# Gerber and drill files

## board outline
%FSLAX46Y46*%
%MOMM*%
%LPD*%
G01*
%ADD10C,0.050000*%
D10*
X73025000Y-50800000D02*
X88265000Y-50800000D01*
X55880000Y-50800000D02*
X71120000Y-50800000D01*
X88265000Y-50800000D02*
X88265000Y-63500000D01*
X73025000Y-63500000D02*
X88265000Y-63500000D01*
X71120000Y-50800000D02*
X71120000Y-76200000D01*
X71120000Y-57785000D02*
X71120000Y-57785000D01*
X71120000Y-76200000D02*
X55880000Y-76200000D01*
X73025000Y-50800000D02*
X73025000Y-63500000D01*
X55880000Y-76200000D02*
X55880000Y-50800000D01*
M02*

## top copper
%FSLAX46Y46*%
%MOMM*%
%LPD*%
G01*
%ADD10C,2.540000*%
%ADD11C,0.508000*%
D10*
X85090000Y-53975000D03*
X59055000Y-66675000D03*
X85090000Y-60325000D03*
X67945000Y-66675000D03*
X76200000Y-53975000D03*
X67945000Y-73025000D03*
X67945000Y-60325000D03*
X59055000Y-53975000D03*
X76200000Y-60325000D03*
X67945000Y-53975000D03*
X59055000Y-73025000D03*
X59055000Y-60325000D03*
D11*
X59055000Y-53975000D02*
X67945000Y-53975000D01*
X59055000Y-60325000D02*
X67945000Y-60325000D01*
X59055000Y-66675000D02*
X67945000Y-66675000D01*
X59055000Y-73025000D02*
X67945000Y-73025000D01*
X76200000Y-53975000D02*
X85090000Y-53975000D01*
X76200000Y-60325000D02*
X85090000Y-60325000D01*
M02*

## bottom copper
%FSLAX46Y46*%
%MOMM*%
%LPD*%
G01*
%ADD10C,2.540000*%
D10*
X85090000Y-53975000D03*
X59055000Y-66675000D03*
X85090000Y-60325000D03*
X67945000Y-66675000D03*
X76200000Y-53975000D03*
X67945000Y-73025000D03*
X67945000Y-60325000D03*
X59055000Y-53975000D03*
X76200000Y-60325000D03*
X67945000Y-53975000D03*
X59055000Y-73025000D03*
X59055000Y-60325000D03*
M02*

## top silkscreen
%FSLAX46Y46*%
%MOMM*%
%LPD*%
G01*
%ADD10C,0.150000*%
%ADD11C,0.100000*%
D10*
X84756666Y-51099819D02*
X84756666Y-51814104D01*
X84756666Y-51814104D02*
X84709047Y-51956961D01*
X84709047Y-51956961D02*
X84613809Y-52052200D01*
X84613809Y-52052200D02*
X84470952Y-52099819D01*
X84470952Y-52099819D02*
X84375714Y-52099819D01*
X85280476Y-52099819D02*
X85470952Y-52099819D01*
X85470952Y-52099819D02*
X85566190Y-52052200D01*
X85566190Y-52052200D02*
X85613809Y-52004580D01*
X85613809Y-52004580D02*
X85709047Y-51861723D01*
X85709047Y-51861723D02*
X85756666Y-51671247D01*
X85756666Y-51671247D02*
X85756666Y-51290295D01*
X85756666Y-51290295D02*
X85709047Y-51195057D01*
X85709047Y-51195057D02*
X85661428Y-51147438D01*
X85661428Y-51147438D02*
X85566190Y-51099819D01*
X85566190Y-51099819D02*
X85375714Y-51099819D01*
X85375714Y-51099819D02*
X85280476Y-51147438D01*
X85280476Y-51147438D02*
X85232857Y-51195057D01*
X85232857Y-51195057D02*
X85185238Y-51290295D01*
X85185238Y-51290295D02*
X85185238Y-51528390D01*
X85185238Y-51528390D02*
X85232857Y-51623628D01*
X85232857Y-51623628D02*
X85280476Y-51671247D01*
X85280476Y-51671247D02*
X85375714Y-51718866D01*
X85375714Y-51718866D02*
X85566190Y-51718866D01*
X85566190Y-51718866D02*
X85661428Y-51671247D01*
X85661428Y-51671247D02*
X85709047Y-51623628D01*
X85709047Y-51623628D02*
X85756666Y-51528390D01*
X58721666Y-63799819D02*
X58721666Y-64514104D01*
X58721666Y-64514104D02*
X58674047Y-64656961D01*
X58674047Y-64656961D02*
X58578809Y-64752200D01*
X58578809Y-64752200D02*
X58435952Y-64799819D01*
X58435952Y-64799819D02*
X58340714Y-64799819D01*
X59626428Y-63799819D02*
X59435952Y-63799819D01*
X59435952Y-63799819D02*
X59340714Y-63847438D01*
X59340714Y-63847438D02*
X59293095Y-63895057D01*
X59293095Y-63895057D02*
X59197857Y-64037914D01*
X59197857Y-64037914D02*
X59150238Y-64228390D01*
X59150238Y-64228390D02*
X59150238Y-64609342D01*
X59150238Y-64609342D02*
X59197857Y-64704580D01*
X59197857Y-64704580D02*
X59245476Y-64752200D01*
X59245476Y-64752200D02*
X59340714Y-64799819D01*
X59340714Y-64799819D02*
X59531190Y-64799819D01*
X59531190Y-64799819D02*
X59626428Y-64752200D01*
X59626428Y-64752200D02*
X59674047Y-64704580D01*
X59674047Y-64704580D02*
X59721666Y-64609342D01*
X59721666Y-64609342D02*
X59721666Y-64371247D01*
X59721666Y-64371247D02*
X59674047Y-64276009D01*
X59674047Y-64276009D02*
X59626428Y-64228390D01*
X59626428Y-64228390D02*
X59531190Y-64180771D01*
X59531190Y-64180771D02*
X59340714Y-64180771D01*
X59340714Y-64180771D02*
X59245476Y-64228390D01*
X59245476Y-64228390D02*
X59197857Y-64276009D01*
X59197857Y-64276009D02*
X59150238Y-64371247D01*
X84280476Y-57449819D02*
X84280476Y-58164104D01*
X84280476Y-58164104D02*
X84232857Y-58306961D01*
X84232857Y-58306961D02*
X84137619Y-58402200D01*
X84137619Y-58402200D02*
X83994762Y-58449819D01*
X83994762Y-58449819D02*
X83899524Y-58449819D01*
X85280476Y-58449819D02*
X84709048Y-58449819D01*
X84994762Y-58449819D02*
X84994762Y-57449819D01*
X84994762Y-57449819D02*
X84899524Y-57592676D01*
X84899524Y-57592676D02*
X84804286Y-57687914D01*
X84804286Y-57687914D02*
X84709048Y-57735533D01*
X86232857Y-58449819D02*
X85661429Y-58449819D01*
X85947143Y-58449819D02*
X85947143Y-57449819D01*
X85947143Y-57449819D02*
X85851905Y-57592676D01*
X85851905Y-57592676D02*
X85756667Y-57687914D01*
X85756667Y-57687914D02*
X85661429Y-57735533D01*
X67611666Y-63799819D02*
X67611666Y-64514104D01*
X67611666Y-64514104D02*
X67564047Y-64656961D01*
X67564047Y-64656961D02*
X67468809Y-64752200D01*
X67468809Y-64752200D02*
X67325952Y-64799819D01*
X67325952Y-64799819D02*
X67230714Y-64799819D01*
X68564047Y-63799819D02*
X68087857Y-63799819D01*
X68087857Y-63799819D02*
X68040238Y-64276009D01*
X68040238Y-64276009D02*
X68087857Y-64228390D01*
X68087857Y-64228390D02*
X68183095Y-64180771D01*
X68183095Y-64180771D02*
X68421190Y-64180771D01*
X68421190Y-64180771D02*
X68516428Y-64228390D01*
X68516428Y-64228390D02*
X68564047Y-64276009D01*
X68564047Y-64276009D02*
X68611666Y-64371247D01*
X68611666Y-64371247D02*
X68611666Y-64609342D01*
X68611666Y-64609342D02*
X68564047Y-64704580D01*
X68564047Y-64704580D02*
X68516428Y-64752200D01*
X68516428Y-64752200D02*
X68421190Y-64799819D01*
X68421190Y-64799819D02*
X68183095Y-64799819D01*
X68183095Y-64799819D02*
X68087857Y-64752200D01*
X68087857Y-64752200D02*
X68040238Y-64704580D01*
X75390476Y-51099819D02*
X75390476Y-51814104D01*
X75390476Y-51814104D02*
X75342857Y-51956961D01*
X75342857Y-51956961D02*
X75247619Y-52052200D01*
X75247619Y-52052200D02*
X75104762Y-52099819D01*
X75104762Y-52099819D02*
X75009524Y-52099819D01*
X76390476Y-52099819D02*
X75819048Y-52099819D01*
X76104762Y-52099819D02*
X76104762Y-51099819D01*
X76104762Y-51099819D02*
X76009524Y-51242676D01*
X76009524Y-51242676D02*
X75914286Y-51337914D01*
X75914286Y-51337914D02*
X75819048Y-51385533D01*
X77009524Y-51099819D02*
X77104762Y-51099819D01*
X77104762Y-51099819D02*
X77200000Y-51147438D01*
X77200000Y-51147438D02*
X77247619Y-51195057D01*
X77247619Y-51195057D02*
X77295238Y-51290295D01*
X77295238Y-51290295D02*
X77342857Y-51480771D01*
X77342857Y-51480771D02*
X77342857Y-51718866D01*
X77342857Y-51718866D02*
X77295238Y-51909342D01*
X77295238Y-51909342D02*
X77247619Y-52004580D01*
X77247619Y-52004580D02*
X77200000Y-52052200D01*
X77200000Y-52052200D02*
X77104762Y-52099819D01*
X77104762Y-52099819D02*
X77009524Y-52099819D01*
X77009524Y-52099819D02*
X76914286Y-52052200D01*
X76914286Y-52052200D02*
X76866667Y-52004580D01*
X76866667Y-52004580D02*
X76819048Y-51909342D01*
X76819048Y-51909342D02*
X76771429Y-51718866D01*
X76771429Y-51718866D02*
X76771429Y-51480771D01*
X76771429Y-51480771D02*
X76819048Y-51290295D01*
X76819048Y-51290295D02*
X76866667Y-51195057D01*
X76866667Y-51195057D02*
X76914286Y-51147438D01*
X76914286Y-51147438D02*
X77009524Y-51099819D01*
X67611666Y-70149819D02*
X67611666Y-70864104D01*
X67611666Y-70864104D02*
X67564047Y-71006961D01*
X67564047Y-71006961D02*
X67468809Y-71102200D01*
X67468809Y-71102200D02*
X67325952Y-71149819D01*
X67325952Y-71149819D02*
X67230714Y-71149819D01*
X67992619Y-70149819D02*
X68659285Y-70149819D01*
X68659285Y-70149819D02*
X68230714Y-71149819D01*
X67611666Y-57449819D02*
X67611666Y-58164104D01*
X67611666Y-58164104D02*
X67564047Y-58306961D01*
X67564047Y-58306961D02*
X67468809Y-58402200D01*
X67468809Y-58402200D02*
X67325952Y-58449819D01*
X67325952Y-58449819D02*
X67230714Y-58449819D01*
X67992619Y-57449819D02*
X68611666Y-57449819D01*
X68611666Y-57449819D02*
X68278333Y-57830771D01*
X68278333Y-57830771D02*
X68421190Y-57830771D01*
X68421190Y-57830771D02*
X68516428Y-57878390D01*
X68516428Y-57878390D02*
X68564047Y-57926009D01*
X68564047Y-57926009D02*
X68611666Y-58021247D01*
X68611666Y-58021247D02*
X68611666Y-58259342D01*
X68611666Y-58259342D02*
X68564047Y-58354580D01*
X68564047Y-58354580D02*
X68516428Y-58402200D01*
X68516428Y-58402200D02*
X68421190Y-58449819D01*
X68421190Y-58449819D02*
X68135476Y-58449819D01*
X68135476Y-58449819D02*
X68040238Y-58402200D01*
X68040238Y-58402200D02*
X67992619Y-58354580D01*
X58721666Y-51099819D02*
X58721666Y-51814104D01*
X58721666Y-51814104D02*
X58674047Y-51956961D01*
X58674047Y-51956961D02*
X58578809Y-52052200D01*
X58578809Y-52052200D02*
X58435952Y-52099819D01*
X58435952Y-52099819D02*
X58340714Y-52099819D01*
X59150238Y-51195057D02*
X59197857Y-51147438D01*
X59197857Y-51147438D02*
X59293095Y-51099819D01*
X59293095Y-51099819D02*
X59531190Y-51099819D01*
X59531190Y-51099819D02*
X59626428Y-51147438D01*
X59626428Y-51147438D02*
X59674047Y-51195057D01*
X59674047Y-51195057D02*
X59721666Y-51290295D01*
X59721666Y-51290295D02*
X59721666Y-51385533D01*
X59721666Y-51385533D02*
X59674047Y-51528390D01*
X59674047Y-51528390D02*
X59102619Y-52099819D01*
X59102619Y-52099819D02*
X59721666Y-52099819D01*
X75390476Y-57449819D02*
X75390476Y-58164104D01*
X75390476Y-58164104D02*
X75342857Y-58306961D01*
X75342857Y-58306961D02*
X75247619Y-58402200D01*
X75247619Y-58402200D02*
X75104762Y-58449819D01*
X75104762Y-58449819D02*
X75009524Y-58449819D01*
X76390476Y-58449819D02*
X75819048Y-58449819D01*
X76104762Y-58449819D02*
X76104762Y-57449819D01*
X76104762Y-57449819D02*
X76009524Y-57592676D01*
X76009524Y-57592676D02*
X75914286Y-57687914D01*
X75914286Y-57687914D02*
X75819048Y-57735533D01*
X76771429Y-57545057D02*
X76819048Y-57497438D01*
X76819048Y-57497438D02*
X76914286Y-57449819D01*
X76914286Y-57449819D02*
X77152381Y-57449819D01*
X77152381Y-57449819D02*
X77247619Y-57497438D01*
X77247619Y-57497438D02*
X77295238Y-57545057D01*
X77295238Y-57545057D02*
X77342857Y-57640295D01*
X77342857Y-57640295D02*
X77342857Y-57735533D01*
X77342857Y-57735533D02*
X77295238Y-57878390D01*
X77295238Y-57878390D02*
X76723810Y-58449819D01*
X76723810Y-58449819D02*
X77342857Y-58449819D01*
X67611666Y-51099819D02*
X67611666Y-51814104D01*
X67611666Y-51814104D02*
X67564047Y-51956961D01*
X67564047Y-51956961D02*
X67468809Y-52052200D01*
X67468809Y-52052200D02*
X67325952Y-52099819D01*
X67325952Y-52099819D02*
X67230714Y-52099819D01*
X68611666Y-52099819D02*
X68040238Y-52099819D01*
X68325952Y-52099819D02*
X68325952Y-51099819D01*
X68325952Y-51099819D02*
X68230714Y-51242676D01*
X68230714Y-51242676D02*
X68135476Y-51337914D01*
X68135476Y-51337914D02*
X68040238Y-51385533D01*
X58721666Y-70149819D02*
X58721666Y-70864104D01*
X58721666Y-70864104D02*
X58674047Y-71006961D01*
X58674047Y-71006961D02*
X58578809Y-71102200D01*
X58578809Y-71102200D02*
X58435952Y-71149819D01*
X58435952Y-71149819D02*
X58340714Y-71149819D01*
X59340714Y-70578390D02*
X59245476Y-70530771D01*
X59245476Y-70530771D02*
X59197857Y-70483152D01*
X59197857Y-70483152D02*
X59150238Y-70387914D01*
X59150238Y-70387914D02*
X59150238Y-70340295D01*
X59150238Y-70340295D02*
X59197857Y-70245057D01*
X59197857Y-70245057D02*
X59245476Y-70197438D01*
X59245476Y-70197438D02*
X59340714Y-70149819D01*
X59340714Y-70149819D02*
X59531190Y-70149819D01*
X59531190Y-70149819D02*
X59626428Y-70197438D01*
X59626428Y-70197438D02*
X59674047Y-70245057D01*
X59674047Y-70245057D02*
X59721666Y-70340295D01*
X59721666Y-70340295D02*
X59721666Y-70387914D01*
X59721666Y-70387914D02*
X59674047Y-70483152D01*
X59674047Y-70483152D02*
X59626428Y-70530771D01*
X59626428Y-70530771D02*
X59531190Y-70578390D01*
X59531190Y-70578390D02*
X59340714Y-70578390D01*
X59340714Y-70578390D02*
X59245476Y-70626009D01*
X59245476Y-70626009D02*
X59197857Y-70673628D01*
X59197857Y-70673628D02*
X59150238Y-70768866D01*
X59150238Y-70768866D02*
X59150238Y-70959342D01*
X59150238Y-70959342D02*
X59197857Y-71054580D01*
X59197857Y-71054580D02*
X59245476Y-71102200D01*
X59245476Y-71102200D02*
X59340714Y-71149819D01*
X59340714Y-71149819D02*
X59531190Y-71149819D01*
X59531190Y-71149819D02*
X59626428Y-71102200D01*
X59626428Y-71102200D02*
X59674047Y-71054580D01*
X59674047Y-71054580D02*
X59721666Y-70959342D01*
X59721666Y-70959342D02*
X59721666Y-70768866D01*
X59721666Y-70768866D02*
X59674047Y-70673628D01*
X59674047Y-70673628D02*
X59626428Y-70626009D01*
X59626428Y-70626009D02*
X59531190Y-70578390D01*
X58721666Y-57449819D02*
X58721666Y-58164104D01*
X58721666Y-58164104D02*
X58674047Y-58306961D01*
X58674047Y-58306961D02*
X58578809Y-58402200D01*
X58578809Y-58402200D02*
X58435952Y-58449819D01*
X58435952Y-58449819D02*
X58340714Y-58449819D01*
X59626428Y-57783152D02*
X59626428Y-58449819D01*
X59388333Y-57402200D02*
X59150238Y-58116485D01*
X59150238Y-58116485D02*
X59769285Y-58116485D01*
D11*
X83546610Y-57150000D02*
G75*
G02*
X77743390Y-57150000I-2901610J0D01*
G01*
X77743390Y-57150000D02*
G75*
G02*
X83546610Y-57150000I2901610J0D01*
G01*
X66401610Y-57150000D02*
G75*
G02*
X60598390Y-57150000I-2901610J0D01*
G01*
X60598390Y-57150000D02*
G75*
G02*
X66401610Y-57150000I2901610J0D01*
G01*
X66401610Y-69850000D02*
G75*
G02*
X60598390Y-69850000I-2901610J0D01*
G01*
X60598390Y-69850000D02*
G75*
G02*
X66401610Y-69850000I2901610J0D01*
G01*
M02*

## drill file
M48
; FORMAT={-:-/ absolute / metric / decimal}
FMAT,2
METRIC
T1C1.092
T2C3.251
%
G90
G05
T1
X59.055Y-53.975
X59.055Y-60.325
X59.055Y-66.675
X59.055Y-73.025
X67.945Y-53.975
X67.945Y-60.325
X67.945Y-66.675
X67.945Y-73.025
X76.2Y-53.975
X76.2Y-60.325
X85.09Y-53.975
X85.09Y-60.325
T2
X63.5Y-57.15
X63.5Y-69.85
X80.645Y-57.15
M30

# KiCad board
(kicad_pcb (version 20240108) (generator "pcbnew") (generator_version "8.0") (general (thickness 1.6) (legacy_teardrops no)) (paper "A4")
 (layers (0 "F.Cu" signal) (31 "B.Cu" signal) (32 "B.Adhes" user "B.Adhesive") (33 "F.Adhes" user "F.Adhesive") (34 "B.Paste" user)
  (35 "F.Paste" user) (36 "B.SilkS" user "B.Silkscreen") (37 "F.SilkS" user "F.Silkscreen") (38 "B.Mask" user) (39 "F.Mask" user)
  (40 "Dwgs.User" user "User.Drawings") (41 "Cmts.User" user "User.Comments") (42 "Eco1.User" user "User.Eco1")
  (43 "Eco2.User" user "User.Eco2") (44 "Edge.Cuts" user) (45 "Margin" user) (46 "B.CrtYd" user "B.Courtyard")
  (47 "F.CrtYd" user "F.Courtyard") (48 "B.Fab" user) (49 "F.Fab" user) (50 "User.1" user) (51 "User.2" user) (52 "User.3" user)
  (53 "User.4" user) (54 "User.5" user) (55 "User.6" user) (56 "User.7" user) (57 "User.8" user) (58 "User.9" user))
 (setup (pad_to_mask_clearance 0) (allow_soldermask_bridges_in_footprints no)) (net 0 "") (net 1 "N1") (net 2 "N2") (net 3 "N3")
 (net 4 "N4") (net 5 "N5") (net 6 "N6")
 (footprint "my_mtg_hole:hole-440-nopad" (layer "F.Cu") (at 80.645 57.15)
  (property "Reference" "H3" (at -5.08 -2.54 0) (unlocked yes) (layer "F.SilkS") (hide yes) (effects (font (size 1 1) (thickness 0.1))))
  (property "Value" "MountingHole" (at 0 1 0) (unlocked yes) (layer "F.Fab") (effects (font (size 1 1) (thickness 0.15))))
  (fp_circle (center 0 0) (end 1.143 2.667) (stroke (width 0.1) (type default)) (fill none) (layer "F.SilkS"))
  (pad "" np_thru_hole circle (at 0 0) (size 1.524 1.524) (drill 3.2512) (layers "F&B.Cu" "*.Mask")))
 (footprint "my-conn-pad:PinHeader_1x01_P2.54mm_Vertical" (layer "F.Cu") (at 85.09 53.975)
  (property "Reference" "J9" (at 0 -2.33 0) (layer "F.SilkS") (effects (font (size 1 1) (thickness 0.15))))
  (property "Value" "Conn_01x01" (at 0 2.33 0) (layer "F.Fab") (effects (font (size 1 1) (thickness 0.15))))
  (pad "1" thru_hole circle (at 0 0) (size 2.54 2.54) (drill 1.0922) (layers "*.Cu" "*.Mask") (remove_unused_layers no) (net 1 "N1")))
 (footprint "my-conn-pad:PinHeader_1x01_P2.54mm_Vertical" (layer "F.Cu") (at 59.055 66.675)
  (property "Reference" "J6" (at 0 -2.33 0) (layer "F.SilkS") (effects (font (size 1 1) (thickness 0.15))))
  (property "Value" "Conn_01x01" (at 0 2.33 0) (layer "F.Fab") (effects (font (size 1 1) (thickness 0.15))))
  (pad "1" thru_hole circle (at 0 0) (size 2.54 2.54) (drill 1.0922) (layers "*.Cu" "*.Mask") (remove_unused_layers no) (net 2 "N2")))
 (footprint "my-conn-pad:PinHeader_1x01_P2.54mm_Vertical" (layer "F.Cu") (at 85.09 60.325)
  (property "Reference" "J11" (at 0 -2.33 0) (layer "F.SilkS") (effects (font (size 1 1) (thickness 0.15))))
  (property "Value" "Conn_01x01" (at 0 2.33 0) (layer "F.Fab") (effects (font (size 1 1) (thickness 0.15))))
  (pad "1" thru_hole circle (at 0 0) (size 2.54 2.54) (drill 1.0922) (layers "*.Cu" "*.Mask") (remove_unused_layers no) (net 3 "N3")))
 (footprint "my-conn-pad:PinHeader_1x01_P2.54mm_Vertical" (layer "F.Cu") (at 67.945 66.675)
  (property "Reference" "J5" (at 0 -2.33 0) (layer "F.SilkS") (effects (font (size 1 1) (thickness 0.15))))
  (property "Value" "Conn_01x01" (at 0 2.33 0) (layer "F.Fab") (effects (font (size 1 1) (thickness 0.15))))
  (pad "1" thru_hole circle (at 0 0) (size 2.54 2.54) (drill 1.0922) (layers "*.Cu" "*.Mask") (remove_unused_layers no) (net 2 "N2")))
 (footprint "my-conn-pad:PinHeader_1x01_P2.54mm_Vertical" (layer "F.Cu") (at 76.2 53.975)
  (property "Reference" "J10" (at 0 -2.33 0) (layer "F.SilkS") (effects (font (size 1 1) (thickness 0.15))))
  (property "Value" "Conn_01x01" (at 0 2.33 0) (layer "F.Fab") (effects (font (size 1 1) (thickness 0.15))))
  (pad "1" thru_hole circle (at 0 0) (size 2.54 2.54) (drill 1.0922) (layers "*.Cu" "*.Mask") (remove_unused_layers no) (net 1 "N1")))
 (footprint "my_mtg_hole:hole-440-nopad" (layer "F.Cu") (at 63.5 57.15)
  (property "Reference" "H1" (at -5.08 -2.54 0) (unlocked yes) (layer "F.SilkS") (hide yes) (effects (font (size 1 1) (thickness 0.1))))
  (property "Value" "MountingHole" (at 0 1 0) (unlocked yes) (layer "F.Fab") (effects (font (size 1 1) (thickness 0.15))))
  (fp_circle (center 0 0) (end 1.143 2.667) (stroke (width 0.1) (type default)) (fill none) (layer "F.SilkS"))
  (pad "" np_thru_hole circle (at 0 0) (size 1.524 1.524) (drill 3.2512) (layers "F&B.Cu" "*.Mask")))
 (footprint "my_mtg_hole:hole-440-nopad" (layer "F.Cu") (at 63.5 69.85)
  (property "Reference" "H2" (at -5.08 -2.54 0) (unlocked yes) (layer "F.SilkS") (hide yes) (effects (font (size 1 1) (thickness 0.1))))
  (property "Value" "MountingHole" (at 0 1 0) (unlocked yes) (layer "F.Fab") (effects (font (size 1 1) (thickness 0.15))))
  (fp_circle (center 0 0) (end 1.143 2.667) (stroke (width 0.1) (type default)) (fill none) (layer "F.SilkS"))
  (pad "" np_thru_hole circle (at 0 0) (size 1.524 1.524) (drill 3.2512) (layers "F&B.Cu" "*.Mask")))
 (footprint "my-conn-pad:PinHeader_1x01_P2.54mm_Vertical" (layer "F.Cu") (at 67.945 73.025)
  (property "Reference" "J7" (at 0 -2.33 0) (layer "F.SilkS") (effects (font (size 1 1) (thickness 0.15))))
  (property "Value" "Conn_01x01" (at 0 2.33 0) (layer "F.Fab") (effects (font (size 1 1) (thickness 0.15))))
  (pad "1" thru_hole circle (at 0 0) (size 2.54 2.54) (drill 1.0922) (layers "*.Cu" "*.Mask") (remove_unused_layers no) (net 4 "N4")))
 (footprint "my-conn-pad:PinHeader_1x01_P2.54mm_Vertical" (layer "F.Cu") (at 67.945 60.325)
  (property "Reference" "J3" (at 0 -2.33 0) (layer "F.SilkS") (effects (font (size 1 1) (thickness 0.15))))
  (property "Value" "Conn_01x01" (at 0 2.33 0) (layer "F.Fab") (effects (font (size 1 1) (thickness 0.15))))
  (pad "1" thru_hole circle (at 0 0) (size 2.54 2.54) (drill 1.0922) (layers "*.Cu" "*.Mask") (remove_unused_layers no) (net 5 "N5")))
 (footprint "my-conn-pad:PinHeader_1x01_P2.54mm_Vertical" (layer "F.Cu") (at 59.055 53.975)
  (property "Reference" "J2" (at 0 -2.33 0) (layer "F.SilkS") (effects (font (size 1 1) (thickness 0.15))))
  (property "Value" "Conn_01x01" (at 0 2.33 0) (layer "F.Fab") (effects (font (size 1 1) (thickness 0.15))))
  (pad "1" thru_hole circle (at 0 0) (size 2.54 2.54) (drill 1.0922) (layers "*.Cu" "*.Mask") (remove_unused_layers no) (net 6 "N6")))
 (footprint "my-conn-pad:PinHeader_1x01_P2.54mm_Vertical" (layer "F.Cu") (at 76.2 60.325)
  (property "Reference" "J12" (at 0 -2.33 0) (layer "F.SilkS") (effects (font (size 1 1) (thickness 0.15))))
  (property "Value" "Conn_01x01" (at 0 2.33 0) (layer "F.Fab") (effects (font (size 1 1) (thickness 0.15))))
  (pad "1" thru_hole circle (at 0 0) (size 2.54 2.54) (drill 1.0922) (layers "*.Cu" "*.Mask") (remove_unused_layers no) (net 3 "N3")))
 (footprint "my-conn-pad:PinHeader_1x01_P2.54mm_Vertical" (layer "F.Cu") (at 67.945 53.975)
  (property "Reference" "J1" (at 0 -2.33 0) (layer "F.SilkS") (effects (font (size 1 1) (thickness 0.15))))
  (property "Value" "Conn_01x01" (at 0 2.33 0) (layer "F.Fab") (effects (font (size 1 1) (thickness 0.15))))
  (pad "1" thru_hole circle (at 0 0) (size 2.54 2.54) (drill 1.0922) (layers "*.Cu" "*.Mask") (remove_unused_layers no) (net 6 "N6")))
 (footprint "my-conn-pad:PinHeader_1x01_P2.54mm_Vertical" (layer "F.Cu") (at 59.055 73.025)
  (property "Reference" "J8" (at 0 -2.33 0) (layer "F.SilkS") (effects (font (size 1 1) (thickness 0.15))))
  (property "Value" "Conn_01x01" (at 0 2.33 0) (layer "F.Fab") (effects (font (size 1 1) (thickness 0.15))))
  (pad "1" thru_hole circle (at 0 0) (size 2.54 2.54) (drill 1.0922) (layers "*.Cu" "*.Mask") (remove_unused_layers no) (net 4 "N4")))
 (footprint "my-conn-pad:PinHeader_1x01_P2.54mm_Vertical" (layer "F.Cu") (at 59.055 60.325)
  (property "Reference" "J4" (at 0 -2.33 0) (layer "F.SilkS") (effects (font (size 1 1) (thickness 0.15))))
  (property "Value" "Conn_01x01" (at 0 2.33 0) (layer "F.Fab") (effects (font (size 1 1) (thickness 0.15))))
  (pad "1" thru_hole circle (at 0 0) (size 2.54 2.54) (drill 1.0922) (layers "*.Cu" "*.Mask") (remove_unused_layers no) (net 5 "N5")))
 (gr_line (start 73.025 50.8) (end 88.265 50.8) (stroke (width 0.05) (type default)) (layer "Edge.Cuts"))
 (gr_line (start 55.88 50.8) (end 71.12 50.8) (stroke (width 0.05) (type default)) (layer "Edge.Cuts"))
 (gr_line (start 88.265 50.8) (end 88.265 63.5) (stroke (width 0.05) (type default)) (layer "Edge.Cuts"))
 (gr_line (start 73.025 63.5) (end 88.265 63.5) (stroke (width 0.05) (type default)) (layer "Edge.Cuts"))
 (gr_line (start 71.12 50.8) (end 71.12 76.2) (stroke (width 0.05) (type default)) (layer "Edge.Cuts"))
 (gr_line (start 71.12 57.785) (end 71.12 57.785) (stroke (width 0.05) (type default)) (layer "Edge.Cuts"))
 (gr_line (start 71.12 76.2) (end 55.88 76.2) (stroke (width 0.05) (type default)) (layer "Edge.Cuts"))
 (gr_line (start 73.025 50.8) (end 73.025 63.5) (stroke (width 0.05) (type default)) (layer "Edge.Cuts"))
 (gr_line (start 55.88 76.2) (end 55.88 50.8) (stroke (width 0.05) (type default)) (layer "Edge.Cuts"))
 (segment (start 59.055 53.975) (end 67.945 53.975) (width 0.508) (layer "F.Cu") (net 6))
 (segment (start 59.055 60.325) (end 67.945 60.325) (width 0.508) (layer "F.Cu") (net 5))
 (segment (start 59.055 66.675) (end 67.945 66.675) (width 0.508) (layer "F.Cu") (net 2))
 (segment (start 59.055 73.025) (end 67.945 73.025) (width 0.508) (layer "F.Cu") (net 4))
 (segment (start 76.2 53.975) (end 85.09 53.975) (width 0.508) (layer "F.Cu") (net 1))
 (segment (start 76.2 60.325) (end 85.09 60.325) (width 0.508) (layer "F.Cu") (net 3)))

